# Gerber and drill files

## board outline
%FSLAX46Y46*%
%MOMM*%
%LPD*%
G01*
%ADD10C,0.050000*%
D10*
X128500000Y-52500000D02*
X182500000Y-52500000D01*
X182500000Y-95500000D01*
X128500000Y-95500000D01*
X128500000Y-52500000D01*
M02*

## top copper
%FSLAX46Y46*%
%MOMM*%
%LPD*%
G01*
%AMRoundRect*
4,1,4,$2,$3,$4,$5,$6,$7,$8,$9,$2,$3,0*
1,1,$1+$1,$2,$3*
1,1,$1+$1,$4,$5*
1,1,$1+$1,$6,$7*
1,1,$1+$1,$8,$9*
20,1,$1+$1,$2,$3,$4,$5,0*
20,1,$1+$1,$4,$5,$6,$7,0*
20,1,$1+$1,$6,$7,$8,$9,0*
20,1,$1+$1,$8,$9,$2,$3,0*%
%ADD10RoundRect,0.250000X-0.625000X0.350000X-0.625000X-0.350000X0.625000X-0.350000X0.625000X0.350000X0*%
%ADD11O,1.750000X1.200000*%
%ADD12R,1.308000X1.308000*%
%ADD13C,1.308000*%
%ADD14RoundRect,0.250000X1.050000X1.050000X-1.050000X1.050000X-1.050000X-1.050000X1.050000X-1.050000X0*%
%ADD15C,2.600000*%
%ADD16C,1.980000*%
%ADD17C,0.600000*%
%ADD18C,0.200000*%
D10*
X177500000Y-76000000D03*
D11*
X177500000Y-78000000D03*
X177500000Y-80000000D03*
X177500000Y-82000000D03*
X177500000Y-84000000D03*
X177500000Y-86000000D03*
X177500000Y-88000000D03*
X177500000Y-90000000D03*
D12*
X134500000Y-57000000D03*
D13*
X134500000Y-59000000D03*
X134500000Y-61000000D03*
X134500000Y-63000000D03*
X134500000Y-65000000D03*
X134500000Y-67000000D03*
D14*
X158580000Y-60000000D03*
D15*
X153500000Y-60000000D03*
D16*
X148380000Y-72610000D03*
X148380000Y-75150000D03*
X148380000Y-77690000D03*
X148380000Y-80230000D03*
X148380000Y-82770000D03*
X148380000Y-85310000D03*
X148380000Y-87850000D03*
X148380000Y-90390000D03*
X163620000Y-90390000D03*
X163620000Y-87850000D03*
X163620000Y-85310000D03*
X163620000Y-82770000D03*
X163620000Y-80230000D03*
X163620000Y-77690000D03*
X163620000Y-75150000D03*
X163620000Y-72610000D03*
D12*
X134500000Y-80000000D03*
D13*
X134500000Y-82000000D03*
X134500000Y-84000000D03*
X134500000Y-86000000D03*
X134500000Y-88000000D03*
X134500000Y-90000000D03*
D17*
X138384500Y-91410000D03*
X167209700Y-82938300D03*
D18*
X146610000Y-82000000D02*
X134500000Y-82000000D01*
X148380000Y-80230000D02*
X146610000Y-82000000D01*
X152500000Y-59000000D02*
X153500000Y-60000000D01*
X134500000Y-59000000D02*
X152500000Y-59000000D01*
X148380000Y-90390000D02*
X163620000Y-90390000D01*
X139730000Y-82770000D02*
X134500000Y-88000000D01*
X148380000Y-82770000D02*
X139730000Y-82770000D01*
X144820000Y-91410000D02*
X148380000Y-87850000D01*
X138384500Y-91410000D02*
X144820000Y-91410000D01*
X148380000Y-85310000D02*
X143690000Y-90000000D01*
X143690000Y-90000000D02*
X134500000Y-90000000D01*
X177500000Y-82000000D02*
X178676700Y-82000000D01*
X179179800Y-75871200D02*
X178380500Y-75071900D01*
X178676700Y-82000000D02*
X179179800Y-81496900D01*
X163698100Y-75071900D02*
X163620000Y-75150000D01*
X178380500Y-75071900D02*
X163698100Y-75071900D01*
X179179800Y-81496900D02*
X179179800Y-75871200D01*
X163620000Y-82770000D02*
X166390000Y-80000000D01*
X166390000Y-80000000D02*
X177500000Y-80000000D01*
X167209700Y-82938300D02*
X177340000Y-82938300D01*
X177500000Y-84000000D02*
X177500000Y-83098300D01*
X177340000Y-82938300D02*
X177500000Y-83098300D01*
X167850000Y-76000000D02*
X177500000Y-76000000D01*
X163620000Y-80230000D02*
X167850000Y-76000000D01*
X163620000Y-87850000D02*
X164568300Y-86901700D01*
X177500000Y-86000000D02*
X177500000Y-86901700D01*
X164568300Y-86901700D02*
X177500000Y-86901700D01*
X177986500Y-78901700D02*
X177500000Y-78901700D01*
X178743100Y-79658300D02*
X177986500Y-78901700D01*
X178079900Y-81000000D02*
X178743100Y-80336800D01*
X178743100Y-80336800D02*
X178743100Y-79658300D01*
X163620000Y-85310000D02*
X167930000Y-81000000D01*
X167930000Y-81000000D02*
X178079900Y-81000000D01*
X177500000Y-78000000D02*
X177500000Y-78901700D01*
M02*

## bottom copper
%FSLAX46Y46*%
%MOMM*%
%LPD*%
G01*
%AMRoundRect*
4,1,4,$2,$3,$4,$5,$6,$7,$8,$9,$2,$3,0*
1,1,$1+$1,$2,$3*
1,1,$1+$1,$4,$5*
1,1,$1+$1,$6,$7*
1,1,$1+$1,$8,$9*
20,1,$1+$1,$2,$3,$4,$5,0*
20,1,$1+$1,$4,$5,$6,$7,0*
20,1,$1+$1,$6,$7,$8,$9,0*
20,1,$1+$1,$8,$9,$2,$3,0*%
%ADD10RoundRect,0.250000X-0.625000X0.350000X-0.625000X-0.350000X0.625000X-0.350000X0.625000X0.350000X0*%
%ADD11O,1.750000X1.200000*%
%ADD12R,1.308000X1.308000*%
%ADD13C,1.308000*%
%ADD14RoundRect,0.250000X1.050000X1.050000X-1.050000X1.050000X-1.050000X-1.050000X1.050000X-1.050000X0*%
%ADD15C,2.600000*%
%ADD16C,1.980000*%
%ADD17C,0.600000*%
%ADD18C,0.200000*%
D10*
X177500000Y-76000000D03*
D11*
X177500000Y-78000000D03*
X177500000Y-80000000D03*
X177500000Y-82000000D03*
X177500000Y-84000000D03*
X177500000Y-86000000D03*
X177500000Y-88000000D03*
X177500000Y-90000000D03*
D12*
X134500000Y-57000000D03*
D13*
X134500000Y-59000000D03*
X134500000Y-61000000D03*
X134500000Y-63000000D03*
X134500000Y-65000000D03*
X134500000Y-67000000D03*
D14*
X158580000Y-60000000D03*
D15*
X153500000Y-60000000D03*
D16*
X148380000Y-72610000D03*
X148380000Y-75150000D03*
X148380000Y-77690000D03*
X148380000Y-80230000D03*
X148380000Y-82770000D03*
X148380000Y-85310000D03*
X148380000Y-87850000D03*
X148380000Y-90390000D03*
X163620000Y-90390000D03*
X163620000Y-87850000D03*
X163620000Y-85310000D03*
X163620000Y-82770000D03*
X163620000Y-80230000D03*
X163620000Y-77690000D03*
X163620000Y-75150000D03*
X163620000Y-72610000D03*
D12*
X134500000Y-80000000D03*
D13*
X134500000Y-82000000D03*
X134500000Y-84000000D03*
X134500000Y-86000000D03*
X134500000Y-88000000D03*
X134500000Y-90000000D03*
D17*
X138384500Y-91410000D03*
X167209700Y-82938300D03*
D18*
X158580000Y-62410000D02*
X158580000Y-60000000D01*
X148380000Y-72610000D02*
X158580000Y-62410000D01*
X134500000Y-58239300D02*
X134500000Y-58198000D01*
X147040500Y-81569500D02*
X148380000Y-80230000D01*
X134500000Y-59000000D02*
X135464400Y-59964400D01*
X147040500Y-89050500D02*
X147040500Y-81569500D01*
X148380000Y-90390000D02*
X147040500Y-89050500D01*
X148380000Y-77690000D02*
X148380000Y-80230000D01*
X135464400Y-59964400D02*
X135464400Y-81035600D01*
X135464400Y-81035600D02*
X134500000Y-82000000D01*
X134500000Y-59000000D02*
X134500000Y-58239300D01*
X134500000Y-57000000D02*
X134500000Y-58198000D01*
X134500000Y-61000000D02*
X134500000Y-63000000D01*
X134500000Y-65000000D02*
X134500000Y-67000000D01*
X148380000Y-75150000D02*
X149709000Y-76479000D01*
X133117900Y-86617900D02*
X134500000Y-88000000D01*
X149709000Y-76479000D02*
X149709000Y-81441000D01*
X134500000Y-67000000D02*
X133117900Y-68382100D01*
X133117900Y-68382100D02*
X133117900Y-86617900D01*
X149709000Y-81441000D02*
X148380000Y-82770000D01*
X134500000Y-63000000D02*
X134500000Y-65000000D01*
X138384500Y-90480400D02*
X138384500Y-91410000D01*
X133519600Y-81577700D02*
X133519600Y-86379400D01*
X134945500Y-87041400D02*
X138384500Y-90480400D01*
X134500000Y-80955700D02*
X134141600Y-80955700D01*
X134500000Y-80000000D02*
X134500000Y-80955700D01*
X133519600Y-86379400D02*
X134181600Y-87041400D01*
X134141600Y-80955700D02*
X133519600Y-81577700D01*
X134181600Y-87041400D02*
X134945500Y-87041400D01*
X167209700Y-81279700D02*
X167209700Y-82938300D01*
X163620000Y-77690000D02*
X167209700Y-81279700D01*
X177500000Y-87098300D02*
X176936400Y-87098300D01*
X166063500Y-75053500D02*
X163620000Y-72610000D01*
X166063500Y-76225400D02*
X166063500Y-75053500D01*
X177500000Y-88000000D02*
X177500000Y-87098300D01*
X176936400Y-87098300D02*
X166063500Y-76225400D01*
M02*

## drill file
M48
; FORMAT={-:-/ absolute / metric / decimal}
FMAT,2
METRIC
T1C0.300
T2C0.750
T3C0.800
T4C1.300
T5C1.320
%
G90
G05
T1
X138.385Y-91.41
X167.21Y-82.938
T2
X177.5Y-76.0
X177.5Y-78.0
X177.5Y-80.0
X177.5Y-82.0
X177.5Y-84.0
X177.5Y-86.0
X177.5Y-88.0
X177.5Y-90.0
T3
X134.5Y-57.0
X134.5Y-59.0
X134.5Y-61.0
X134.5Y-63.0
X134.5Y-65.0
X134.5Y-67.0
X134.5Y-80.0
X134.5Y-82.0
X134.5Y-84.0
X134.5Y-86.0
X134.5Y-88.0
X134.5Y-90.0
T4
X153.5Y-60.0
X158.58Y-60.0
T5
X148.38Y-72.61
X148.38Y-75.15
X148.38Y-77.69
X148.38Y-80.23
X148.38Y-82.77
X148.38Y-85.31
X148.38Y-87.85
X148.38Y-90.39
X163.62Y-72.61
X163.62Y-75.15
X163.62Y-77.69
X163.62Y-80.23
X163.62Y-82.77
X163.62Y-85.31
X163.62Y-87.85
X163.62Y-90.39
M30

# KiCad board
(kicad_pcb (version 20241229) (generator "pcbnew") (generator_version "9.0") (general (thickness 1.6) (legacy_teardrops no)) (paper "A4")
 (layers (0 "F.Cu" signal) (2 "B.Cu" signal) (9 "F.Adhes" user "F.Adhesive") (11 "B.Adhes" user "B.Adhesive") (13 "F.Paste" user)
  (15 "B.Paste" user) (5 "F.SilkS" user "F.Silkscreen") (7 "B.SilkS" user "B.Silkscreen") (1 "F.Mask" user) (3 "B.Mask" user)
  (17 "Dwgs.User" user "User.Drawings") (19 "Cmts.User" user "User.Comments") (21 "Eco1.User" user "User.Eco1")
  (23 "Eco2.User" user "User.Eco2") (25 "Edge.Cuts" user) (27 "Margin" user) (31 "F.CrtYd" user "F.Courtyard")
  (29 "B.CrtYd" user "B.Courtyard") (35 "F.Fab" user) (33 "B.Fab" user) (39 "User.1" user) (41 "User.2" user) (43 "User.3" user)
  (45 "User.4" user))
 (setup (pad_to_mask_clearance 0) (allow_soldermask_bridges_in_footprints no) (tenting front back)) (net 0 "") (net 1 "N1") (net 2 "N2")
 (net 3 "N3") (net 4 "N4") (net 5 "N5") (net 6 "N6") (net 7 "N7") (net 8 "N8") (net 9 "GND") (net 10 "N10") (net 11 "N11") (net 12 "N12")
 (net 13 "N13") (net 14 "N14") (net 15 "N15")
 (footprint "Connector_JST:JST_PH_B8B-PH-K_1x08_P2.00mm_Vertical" (layer "F.Cu") (at 177.5 76 -90)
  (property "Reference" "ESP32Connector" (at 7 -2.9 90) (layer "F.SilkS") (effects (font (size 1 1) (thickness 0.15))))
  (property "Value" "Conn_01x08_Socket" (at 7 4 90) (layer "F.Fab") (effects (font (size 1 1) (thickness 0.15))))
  (pad "1" thru_hole roundrect (at 0 0 270) (size 1.2 1.75) (drill 0.75) (layers "*.Cu" "*.Mask") (remove_unused_layers no)
   (roundrect_rratio 0.208333) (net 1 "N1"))
  (pad "2" thru_hole oval (at 2 0 270) (size 1.2 1.75) (drill 0.75) (layers "*.Cu" "*.Mask") (remove_unused_layers no) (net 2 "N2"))
  (pad "3" thru_hole oval (at 4 0 270) (size 1.2 1.75) (drill 0.75) (layers "*.Cu" "*.Mask") (remove_unused_layers no) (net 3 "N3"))
  (pad "4" thru_hole oval (at 6 0 270) (size 1.2 1.75) (drill 0.75) (layers "*.Cu" "*.Mask") (remove_unused_layers no) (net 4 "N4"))
  (pad "5" thru_hole oval (at 8 0 270) (size 1.2 1.75) (drill 0.75) (layers "*.Cu" "*.Mask") (remove_unused_layers no) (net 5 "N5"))
  (pad "6" thru_hole oval (at 10 0 270) (size 1.2 1.75) (drill 0.75) (layers "*.Cu" "*.Mask") (remove_unused_layers no) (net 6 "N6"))
  (pad "7" thru_hole oval (at 12 0 270) (size 1.2 1.75) (drill 0.75) (layers "*.Cu" "*.Mask") (remove_unused_layers no) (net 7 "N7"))
  (pad "8" thru_hole oval (at 14 0 270) (size 1.2 1.75) (drill 0.75) (layers "*.Cu" "*.Mask") (remove_unused_layers no) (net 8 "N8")))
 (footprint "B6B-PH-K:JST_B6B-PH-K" (layer "F.Cu") (at 133.95 62 90)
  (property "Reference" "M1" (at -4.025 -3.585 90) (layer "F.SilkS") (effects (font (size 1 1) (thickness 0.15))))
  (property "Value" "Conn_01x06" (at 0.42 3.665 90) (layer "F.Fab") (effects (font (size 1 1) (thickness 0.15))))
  (pad "1" thru_hole rect (at 5 0.55 90) (size 1.308 1.308) (drill 0.8) (layers "*.Cu" "*.Mask") (remove_unused_layers no) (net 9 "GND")
   (solder_mask_margin 0.102))
  (pad "2" thru_hole circle (at 3 0.55 90) (size 1.308 1.308) (drill 0.8) (layers "*.Cu" "*.Mask") (remove_unused_layers no) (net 9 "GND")
   (solder_mask_margin 0.102))
  (pad "3" thru_hole circle (at 1 0.55 90) (size 1.308 1.308) (drill 0.8) (layers "*.Cu" "*.Mask") (remove_unused_layers no) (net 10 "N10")
   (solder_mask_margin 0.102))
  (pad "4" thru_hole circle (at -1 0.55 90) (size 1.308 1.308) (drill 0.8) (layers "*.Cu" "*.Mask") (remove_unused_layers no) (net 10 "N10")
   (solder_mask_margin 0.102))
  (pad "5" thru_hole circle (at -3 0.55 90) (size 1.308 1.308) (drill 0.8) (layers "*.Cu" "*.Mask") (remove_unused_layers no) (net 10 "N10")
   (solder_mask_margin 0.102))
  (pad "6" thru_hole circle (at -5 0.55 90) (size 1.308 1.308) (drill 0.8) (layers "*.Cu" "*.Mask") (remove_unused_layers no) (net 10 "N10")
   (solder_mask_margin 0.102)))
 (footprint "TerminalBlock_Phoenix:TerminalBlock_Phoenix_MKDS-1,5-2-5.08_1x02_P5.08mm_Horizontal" (layer "F.Cu") (at 158.58 60 180)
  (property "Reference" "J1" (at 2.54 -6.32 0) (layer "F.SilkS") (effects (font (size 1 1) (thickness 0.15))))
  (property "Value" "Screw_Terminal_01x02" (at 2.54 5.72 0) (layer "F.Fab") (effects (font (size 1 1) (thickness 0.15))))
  (pad "1" thru_hole roundrect (at 0 0 180) (size 2.6 2.6) (drill 1.3) (layers "*.Cu" "*.Mask") (remove_unused_layers no)
   (roundrect_rratio 0.096154) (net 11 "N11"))
  (pad "2" thru_hole circle (at 5.08 0 180) (size 2.6 2.6) (drill 1.3) (layers "*.Cu" "*.Mask") (remove_unused_layers no) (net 9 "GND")))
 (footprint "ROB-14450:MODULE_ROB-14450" (layer "F.Cu") (at 156 81.5)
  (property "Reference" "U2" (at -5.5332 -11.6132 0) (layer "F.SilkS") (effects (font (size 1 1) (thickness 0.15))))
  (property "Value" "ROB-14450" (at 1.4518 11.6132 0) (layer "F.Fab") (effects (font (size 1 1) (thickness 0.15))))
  (pad "1" thru_hole circle (at -7.62 -8.89) (size 1.98 1.98) (drill 1.32) (layers "*.Cu" "*.Mask") (remove_unused_layers no) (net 11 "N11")
   (solder_mask_margin 0.102))
  (pad "2" thru_hole circle (at -7.62 -6.35) (size 1.98 1.98) (drill 1.32) (layers "*.Cu" "*.Mask") (remove_unused_layers no) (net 10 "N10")
   (solder_mask_margin 0.102))
  (pad "3" thru_hole circle (at -7.62 -3.81) (size 1.98 1.98) (drill 1.32) (layers "*.Cu" "*.Mask") (remove_unused_layers no) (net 9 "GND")
   (solder_mask_margin 0.102))
  (pad "4" thru_hole circle (at -7.62 -1.27) (size 1.98 1.98) (drill 1.32) (layers "*.Cu" "*.Mask") (remove_unused_layers no) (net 9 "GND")
   (solder_mask_margin 0.102))
  (pad "5" thru_hole circle (at -7.62 1.27) (size 1.98 1.98) (drill 1.32) (layers "*.Cu" "*.Mask") (remove_unused_layers no) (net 10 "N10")
   (solder_mask_margin 0.102))
  (pad "6" thru_hole circle (at -7.62 3.81) (size 1.98 1.98) (drill 1.32) (layers "*.Cu" "*.Mask") (remove_unused_layers no) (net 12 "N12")
   (solder_mask_margin 0.102))
  (pad "7" thru_hole circle (at -7.62 6.35) (size 1.98 1.98) (drill 1.32) (layers "*.Cu" "*.Mask") (remove_unused_layers no) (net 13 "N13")
   (solder_mask_margin 0.102))
  (pad "8" thru_hole circle (at -7.62 8.89) (size 1.98 1.98) (drill 1.32) (layers "*.Cu" "*.Mask") (remove_unused_layers no) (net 9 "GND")
   (solder_mask_margin 0.102))
  (pad "9" thru_hole circle (at 7.62 8.89) (size 1.98 1.98) (drill 1.32) (layers "*.Cu" "*.Mask") (remove_unused_layers no) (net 9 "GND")
   (solder_mask_margin 0.102))
  (pad "10" thru_hole circle (at 7.62 6.35) (size 1.98 1.98) (drill 1.32) (layers "*.Cu" "*.Mask") (remove_unused_layers no) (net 6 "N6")
   (solder_mask_margin 0.102))
  (pad "11" thru_hole circle (at 7.62 3.81) (size 1.98 1.98) (drill 1.32) (layers "*.Cu" "*.Mask") (remove_unused_layers no) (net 2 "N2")
   (solder_mask_margin 0.102))
  (pad "12" thru_hole circle (at 7.62 1.27) (size 1.98 1.98) (drill 1.32) (layers "*.Cu" "*.Mask") (remove_unused_layers no) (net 3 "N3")
   (solder_mask_margin 0.102))
  (pad "13" thru_hole circle (at 7.62 -1.27) (size 1.98 1.98) (drill 1.32) (layers "*.Cu" "*.Mask") (remove_unused_layers no) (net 1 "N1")
   (solder_mask_margin 0.102))
  (pad "14" thru_hole circle (at 7.62 -3.81) (size 1.98 1.98) (drill 1.32) (layers "*.Cu" "*.Mask") (remove_unused_layers no) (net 5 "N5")
   (solder_mask_margin 0.102))
  (pad "15" thru_hole circle (at 7.62 -6.35) (size 1.98 1.98) (drill 1.32) (layers "*.Cu" "*.Mask") (remove_unused_layers no) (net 4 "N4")
   (solder_mask_margin 0.102))
  (pad "16" thru_hole circle (at 7.62 -8.89) (size 1.98 1.98) (drill 1.32) (layers "*.Cu" "*.Mask") (remove_unused_layers no) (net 7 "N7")
   (solder_mask_margin 0.102)))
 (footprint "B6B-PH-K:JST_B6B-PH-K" (layer "F.Cu") (at 133.95 85 90)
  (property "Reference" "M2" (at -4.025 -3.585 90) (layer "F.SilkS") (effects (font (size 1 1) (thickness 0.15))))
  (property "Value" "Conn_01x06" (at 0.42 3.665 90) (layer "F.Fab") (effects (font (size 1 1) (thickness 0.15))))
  (pad "1" thru_hole rect (at 5 0.55 90) (size 1.308 1.308) (drill 0.8) (layers "*.Cu" "*.Mask") (remove_unused_layers no) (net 13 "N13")
   (solder_mask_margin 0.102))
  (pad "2" thru_hole circle (at 3 0.55 90) (size 1.308 1.308) (drill 0.8) (layers "*.Cu" "*.Mask") (remove_unused_layers no) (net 9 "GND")
   (solder_mask_margin 0.102))
  (pad "3" thru_hole circle (at 1 0.55 90) (size 1.308 1.308) (drill 0.8) (layers "*.Cu" "*.Mask") (remove_unused_layers no) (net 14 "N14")
   (solder_mask_margin 0.102))
  (pad "4" thru_hole circle (at -1 0.55 90) (size 1.308 1.308) (drill 0.8) (layers "*.Cu" "*.Mask") (remove_unused_layers no) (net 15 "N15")
   (solder_mask_margin 0.102))
  (pad "5" thru_hole circle (at -3 0.55 90) (size 1.308 1.308) (drill 0.8) (layers "*.Cu" "*.Mask") (remove_unused_layers no) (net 10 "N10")
   (solder_mask_margin 0.102))
  (pad "6" thru_hole circle (at -5 0.55 90) (size 1.308 1.308) (drill 0.8) (layers "*.Cu" "*.Mask") (remove_unused_layers no) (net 12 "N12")
   (solder_mask_margin 0.102)))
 (gr_rect (start 128.5 52.5) (end 182.5 95.5) (stroke (width 0.05) (type default)) (fill no) (layer "Edge.Cuts"))
 (segment (start 158.58 62.41) (end 158.58 60) (width 0.2) (layer "B.Cu") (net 11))
 (segment (start 148.38 72.61) (end 158.58 62.41) (width 0.2) (layer "B.Cu") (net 11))
 (segment (start 146.61 82) (end 134.5 82) (width 0.2) (layer "F.Cu") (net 9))
 (segment (start 148.38 80.23) (end 146.61 82) (width 0.2) (layer "F.Cu") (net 9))
 (segment (start 152.5 59) (end 153.5 60) (width 0.2) (layer "F.Cu") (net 9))
 (segment (start 134.5 59) (end 152.5 59) (width 0.2) (layer "F.Cu") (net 9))
 (segment (start 148.38 90.39) (end 163.62 90.39) (width 0.2) (layer "F.Cu") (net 9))
 (segment (start 134.5 58.2393) (end 134.5 58.198) (width 0.2) (layer "B.Cu") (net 9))
 (segment (start 147.0405 81.5695) (end 148.38 80.23) (width 0.2) (layer "B.Cu") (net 9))
 (segment (start 134.5 59) (end 135.4644 59.9644) (width 0.2) (layer "B.Cu") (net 9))
 (segment (start 147.0405 89.0505) (end 147.0405 81.5695) (width 0.2) (layer "B.Cu") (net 9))
 (segment (start 148.38 90.39) (end 147.0405 89.0505) (width 0.2) (layer "B.Cu") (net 9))
 (segment (start 148.38 77.69) (end 148.38 80.23) (width 0.2) (layer "B.Cu") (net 9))
 (segment (start 135.4644 59.9644) (end 135.4644 81.0356) (width 0.2) (layer "B.Cu") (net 9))
 (segment (start 135.4644 81.0356) (end 134.5 82) (width 0.2) (layer "B.Cu") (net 9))
 (segment (start 134.5 59) (end 134.5 58.2393) (width 0.2) (layer "B.Cu") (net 9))
 (segment (start 134.5 57) (end 134.5 58.198) (width 0.2) (layer "B.Cu") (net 9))
 (segment (start 139.73 82.77) (end 134.5 88) (width 0.2) (layer "F.Cu") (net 10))
 (segment (start 148.38 82.77) (end 139.73 82.77) (width 0.2) (layer "F.Cu") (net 10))
 (segment (start 134.5 61) (end 134.5 63) (width 0.2) (layer "B.Cu") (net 10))
 (segment (start 134.5 65) (end 134.5 67) (width 0.2) (layer "B.Cu") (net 10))
 (segment (start 148.38 75.15) (end 149.709 76.479) (width 0.2) (layer "B.Cu") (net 10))
 (segment (start 133.1179 86.6179) (end 134.5 88) (width 0.2) (layer "B.Cu") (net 10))
 (segment (start 149.709 76.479) (end 149.709 81.441) (width 0.2) (layer "B.Cu") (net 10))
 (segment (start 134.5 67) (end 133.1179 68.3821) (width 0.2) (layer "B.Cu") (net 10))
 (segment (start 133.1179 68.3821) (end 133.1179 86.6179) (width 0.2) (layer "B.Cu") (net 10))
 (segment (start 149.709 81.441) (end 148.38 82.77) (width 0.2) (layer "B.Cu") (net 10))
 (segment (start 134.5 63) (end 134.5 65) (width 0.2) (layer "B.Cu") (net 10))
 (segment (start 144.82 91.41) (end 148.38 87.85) (width 0.2) (layer "F.Cu") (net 13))
 (segment (start 138.3845 91.41) (end 144.82 91.41) (width 0.2) (layer "F.Cu") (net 13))
 (via (at 138.3845 91.41) (size 0.6) (drill 0.3) (layers "F.Cu" "B.Cu") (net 13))
 (segment (start 138.3845 90.4804) (end 138.3845 91.41) (width 0.2) (layer "B.Cu") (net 13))
 (segment (start 133.5196 81.5777) (end 133.5196 86.3794) (width 0.2) (layer "B.Cu") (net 13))
 (segment (start 134.9455 87.0414) (end 138.3845 90.4804) (width 0.2) (layer "B.Cu") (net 13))
 (segment (start 134.5 80.9557) (end 134.1416 80.9557) (width 0.2) (layer "B.Cu") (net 13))
 (segment (start 134.5 80) (end 134.5 80.9557) (width 0.2) (layer "B.Cu") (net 13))
 (segment (start 133.5196 86.3794) (end 134.1816 87.0414) (width 0.2) (layer "B.Cu") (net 13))
 (segment (start 134.1416 80.9557) (end 133.5196 81.5777) (width 0.2) (layer "B.Cu") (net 13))
 (segment (start 134.1816 87.0414) (end 134.9455 87.0414) (width 0.2) (layer "B.Cu") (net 13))
 (segment (start 148.38 85.31) (end 143.69 90) (width 0.2) (layer "F.Cu") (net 12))
 (segment (start 143.69 90) (end 134.5 90) (width 0.2) (layer "F.Cu") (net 12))
 (segment (start 177.5 82) (end 178.6767 82) (width 0.2) (layer "F.Cu") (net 4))
 (segment (start 179.1798 75.8712) (end 178.3805 75.0719) (width 0.2) (layer "F.Cu") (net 4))
 (segment (start 178.6767 82) (end 179.1798 81.4969) (width 0.2) (layer "F.Cu") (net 4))
 (segment (start 163.6981 75.0719) (end 163.62 75.15) (width 0.2) (layer "F.Cu") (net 4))
 (segment (start 178.3805 75.0719) (end 163.6981 75.0719) (width 0.2) (layer "F.Cu") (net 4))
 (segment (start 179.1798 81.4969) (end 179.1798 75.8712) (width 0.2) (layer "F.Cu") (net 4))
 (segment (start 163.62 82.77) (end 166.39 80) (width 0.2) (layer "F.Cu") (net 3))
 (segment (start 166.39 80) (end 177.5 80) (width 0.2) (layer "F.Cu") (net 3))
 (segment (start 167.2097 82.9383) (end 177.34 82.9383) (width 0.2) (layer "F.Cu") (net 5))
 (segment (start 177.5 84) (end 177.5 83.0983) (width 0.2) (layer "F.Cu") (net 5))
 (segment (start 177.34 82.9383) (end 177.5 83.0983) (width 0.2) (layer "F.Cu") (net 5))
 (via (at 167.2097 82.9383) (size 0.6) (drill 0.3) (layers "F.Cu" "B.Cu") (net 5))
 (segment (start 167.2097 81.2797) (end 167.2097 82.9383) (width 0.2) (layer "B.Cu") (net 5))
 (segment (start 163.62 77.69) (end 167.2097 81.2797) (width 0.2) (layer "B.Cu") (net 5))
 (segment (start 167.85 76) (end 177.5 76) (width 0.2) (layer "F.Cu") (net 1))
 (segment (start 163.62 80.23) (end 167.85 76) (width 0.2) (layer "F.Cu") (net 1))
 (segment (start 177.5 87.0983) (end 176.9364 87.0983) (width 0.2) (layer "B.Cu") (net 7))
 (segment (start 166.0635 75.0535) (end 163.62 72.61) (width 0.2) (layer "B.Cu") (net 7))
 (segment (start 166.0635 76.2254) (end 166.0635 75.0535) (width 0.2) (layer "B.Cu") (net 7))
 (segment (start 177.5 88) (end 177.5 87.0983) (width 0.2) (layer "B.Cu") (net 7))
 (segment (start 176.9364 87.0983) (end 166.0635 76.2254) (width 0.2) (layer "B.Cu") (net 7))
 (segment (start 163.62 87.85) (end 164.5683 86.9017) (width 0.2) (layer "F.Cu") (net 6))
 (segment (start 177.5 86) (end 177.5 86.9017) (width 0.2) (layer "F.Cu") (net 6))
 (segment (start 164.5683 86.9017) (end 177.5 86.9017) (width 0.2) (layer "F.Cu") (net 6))
 (segment (start 177.9865 78.9017) (end 177.5 78.9017) (width 0.2) (layer "F.Cu") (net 2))
 (segment (start 178.7431 79.6583) (end 177.9865 78.9017) (width 0.2) (layer "F.Cu") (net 2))
 (segment (start 178.0799 81) (end 178.7431 80.3368) (width 0.2) (layer "F.Cu") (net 2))
 (segment (start 178.7431 80.3368) (end 178.7431 79.6583) (width 0.2) (layer "F.Cu") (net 2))
 (segment (start 163.62 85.31) (end 167.93 81) (width 0.2) (layer "F.Cu") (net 2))
 (segment (start 167.93 81) (end 178.0799 81) (width 0.2) (layer "F.Cu") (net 2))
 (segment (start 177.5 78) (end 177.5 78.9017) (width 0.2) (layer "F.Cu") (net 2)))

